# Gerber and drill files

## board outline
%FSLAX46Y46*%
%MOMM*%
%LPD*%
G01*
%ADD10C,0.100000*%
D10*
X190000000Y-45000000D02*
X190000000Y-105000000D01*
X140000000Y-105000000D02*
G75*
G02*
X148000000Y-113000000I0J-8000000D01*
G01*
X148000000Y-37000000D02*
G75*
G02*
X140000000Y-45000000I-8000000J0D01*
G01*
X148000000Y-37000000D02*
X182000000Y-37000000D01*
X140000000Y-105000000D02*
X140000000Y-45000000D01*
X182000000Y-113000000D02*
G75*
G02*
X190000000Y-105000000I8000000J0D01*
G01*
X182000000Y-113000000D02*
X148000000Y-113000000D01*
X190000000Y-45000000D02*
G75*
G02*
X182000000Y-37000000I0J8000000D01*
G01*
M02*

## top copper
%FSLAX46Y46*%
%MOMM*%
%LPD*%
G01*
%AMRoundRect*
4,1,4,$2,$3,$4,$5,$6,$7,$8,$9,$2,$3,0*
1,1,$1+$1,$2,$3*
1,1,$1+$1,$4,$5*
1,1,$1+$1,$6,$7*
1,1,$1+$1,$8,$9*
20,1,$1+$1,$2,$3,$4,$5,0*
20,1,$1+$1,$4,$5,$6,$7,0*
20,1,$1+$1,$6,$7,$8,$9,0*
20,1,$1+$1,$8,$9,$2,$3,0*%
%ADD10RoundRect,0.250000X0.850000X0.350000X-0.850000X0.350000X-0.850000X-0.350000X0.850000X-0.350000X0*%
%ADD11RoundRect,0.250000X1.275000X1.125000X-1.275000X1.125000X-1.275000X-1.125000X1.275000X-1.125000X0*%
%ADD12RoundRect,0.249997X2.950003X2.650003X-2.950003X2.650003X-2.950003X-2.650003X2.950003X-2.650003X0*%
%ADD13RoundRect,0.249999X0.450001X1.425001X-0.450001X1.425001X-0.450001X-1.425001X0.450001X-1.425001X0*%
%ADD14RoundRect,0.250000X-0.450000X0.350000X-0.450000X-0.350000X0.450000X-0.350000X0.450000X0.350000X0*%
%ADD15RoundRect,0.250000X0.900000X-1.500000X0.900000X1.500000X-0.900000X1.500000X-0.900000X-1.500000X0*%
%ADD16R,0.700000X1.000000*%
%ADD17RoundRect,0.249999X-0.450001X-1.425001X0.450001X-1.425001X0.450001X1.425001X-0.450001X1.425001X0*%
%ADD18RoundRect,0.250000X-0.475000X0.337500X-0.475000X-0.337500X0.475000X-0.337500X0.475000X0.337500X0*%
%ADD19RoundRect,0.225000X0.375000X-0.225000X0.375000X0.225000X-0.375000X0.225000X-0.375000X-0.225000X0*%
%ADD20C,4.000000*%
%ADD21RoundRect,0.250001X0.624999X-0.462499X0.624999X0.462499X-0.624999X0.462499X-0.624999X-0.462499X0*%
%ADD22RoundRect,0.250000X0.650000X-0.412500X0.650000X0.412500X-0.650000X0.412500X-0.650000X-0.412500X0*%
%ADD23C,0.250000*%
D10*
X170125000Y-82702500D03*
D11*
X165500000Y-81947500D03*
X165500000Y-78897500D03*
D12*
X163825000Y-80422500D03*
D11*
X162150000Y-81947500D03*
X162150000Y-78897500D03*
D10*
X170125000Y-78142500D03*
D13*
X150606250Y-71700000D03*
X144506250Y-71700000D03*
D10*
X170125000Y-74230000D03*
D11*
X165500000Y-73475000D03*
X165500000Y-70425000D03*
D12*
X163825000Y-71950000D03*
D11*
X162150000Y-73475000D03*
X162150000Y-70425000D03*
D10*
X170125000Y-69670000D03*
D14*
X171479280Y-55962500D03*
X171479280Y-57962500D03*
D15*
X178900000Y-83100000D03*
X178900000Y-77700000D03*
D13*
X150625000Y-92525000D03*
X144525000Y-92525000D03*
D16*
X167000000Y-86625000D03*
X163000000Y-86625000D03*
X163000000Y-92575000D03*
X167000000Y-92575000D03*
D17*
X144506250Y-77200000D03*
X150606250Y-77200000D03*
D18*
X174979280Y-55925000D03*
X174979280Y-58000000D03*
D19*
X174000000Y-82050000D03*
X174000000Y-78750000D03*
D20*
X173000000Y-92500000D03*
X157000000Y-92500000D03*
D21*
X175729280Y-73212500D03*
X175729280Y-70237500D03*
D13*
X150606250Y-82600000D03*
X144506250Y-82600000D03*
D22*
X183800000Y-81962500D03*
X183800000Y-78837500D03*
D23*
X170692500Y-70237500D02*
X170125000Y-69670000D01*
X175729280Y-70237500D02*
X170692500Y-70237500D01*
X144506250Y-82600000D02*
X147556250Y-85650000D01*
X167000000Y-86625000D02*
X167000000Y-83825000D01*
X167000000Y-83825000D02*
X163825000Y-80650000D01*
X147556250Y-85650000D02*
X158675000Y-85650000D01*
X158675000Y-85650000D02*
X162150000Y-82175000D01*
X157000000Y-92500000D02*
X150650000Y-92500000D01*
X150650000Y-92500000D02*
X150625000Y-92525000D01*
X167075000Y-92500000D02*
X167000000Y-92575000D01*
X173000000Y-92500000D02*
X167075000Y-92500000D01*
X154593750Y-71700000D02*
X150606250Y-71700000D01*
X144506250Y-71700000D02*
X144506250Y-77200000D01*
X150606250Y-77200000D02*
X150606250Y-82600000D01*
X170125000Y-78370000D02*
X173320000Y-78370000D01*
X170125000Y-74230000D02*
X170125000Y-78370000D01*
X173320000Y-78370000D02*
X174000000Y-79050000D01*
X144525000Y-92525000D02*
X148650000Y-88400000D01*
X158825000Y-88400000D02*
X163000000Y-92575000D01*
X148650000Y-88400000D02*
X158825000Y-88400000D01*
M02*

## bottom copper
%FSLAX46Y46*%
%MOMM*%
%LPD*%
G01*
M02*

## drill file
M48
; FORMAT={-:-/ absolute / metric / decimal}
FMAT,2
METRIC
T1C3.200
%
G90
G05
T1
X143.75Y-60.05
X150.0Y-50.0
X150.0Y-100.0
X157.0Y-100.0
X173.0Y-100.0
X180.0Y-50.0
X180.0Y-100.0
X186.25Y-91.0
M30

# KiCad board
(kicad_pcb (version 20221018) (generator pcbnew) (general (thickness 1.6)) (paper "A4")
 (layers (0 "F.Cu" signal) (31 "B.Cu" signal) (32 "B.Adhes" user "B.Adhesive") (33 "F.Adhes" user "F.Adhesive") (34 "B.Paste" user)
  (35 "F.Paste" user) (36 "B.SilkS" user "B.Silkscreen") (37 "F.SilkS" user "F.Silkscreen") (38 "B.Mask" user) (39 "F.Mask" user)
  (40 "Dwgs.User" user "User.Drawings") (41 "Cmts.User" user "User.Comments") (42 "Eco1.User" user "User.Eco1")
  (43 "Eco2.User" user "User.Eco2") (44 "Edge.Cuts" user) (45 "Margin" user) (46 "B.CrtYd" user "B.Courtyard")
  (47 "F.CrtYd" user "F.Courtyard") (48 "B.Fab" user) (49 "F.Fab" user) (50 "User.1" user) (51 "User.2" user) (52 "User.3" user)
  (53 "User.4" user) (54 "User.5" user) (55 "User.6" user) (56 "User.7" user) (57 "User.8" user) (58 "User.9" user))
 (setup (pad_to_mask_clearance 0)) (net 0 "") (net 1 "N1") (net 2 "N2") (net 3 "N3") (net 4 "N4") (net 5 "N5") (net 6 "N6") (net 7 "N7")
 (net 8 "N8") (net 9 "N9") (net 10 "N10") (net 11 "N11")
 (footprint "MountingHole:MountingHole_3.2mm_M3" (layer "F.Cu") (at 186.25 91)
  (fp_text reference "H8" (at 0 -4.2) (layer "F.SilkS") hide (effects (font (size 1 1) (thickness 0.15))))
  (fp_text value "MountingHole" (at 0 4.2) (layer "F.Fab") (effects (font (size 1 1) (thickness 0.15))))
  (pad "" np_thru_hole circle (at 0 0) (size 3.2 3.2) (drill 3.2) (layers "*.Cu" "*.Mask")))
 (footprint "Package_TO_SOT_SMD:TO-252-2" (layer "F.Cu") (at 165.085 80.4225 180)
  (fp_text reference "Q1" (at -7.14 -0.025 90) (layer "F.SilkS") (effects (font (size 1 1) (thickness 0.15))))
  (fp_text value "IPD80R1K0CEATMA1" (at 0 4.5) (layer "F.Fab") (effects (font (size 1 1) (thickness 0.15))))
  (pad "1" smd roundrect (at -5.04 -2.28 180) (size 2.2 1.2) (layers "F.Cu" "F.Paste" "F.Mask") (roundrect_rratio 0.2083333333) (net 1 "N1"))
  (pad "2" smd roundrect (at -0.415 -1.525 180) (size 3.05 2.75) (layers "F.Cu" "F.Paste") (roundrect_rratio 0.09090909091) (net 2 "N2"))
  (pad "2" smd roundrect (at -0.415 1.525 180) (size 3.05 2.75) (layers "F.Cu" "F.Paste") (roundrect_rratio 0.09090909091) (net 2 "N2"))
  (pad "2" smd roundrect (at 1.26 0 180) (size 6.4 5.8) (layers "F.Cu" "F.Mask") (roundrect_rratio 0.04310293103) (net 2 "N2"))
  (pad "2" smd roundrect (at 2.935 -1.525 180) (size 3.05 2.75) (layers "F.Cu" "F.Paste") (roundrect_rratio 0.09090909091) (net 2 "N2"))
  (pad "2" smd roundrect (at 2.935 1.525 180) (size 3.05 2.75) (layers "F.Cu" "F.Paste") (roundrect_rratio 0.09090909091) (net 2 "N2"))
  (pad "3" smd roundrect (at -5.04 2.28 180) (size 2.2 1.2) (layers "F.Cu" "F.Paste" "F.Mask") (roundrect_rratio 0.2083333333) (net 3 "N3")))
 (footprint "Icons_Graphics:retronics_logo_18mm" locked (layer "F.Cu") (at 165 105)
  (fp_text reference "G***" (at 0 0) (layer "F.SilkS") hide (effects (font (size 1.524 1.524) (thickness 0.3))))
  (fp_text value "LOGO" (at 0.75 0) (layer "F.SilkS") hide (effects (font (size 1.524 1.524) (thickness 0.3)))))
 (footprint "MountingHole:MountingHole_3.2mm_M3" (layer "F.Cu") (at 150 100)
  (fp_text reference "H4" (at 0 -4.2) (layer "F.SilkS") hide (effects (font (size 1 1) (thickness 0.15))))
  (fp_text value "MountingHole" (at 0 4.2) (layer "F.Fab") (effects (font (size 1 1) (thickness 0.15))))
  (pad "" np_thru_hole circle (at 0 0) (size 3.2 3.2) (drill 3.2) (layers "*.Cu" "*.Mask")))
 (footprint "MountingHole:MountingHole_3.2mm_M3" (layer "F.Cu") (at 180 50)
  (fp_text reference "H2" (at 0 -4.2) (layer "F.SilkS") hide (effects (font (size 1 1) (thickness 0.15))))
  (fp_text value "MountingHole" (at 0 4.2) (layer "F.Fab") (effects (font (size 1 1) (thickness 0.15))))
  (pad "" np_thru_hole circle (at 0 0) (size 3.2 3.2) (drill 3.2) (layers "*.Cu" "*.Mask")))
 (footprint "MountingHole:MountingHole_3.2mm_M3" (layer "F.Cu") (at 157 100)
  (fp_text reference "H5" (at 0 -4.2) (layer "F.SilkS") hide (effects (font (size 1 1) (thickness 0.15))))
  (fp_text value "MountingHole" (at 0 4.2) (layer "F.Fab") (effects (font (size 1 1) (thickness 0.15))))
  (pad "" np_thru_hole circle (at 0 0) (size 3.2 3.2) (drill 3.2) (layers "*.Cu" "*.Mask")))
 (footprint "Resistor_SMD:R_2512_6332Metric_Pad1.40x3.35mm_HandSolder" (layer "F.Cu") (at 147.55625 71.7 180)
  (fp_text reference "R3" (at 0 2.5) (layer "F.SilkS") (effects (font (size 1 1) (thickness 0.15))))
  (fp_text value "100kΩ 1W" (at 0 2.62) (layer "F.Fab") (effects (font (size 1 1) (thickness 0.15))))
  (pad "1" smd roundrect (at -3.05 0 180) (size 1.4 3.35) (layers "F.Cu" "F.Paste" "F.Mask") (roundrect_rratio 0.1785707143) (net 1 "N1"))
  (pad "2" smd roundrect (at 3.05 0 180) (size 1.4 3.35) (layers "F.Cu" "F.Paste" "F.Mask") (roundrect_rratio 0.1785707143) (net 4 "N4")))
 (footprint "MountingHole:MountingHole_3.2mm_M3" (layer "F.Cu") (at 180 100)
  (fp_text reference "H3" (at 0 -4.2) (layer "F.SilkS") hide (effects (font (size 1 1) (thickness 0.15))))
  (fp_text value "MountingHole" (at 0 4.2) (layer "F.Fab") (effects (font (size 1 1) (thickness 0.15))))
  (pad "" np_thru_hole circle (at 0 0) (size 3.2 3.2) (drill 3.2) (layers "*.Cu" "*.Mask")))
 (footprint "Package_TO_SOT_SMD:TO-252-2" (layer "F.Cu") (at 165.085 71.95 180)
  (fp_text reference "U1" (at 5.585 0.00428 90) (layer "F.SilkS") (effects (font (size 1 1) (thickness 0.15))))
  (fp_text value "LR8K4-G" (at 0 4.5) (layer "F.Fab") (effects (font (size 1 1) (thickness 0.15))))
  (pad "1" smd roundrect (at -5.04 -2.28 180) (size 2.2 1.2) (layers "F.Cu" "F.Paste" "F.Mask") (roundrect_rratio 0.2083333333) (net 3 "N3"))
  (pad "2" smd roundrect (at -0.415 -1.525 180) (size 3.05 2.75) (layers "F.Cu" "F.Paste") (roundrect_rratio 0.09090909091) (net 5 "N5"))
  (pad "2" smd roundrect (at -0.415 1.525 180) (size 3.05 2.75) (layers "F.Cu" "F.Paste") (roundrect_rratio 0.09090909091) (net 5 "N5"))
  (pad "2" smd roundrect (at 1.26 0 180) (size 6.4 5.8) (layers "F.Cu" "F.Mask") (roundrect_rratio 0.04310293103) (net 5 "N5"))
  (pad "2" smd roundrect (at 2.935 -1.525 180) (size 3.05 2.75) (layers "F.Cu" "F.Paste") (roundrect_rratio 0.09090909091) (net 5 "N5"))
  (pad "2" smd roundrect (at 2.935 1.525 180) (size 3.05 2.75) (layers "F.Cu" "F.Paste") (roundrect_rratio 0.09090909091) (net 5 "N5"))
  (pad "3" smd roundrect (at -5.04 2.28 180) (size 2.2 1.2) (layers "F.Cu" "F.Paste" "F.Mask") (roundrect_rratio 0.2083333333) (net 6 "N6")))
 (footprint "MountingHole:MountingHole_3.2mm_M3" (layer "F.Cu") (at 143.75 60.05)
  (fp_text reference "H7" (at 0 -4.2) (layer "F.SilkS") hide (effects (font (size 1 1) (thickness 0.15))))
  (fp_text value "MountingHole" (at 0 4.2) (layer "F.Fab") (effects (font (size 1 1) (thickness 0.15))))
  (pad "" np_thru_hole circle (at 0 0) (size 3.2 3.2) (drill 3.2) (layers "*.Cu" "*.Mask")))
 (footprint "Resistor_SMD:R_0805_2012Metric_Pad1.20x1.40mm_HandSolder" (layer "F.Cu") (at 171.47928 56.9625 -90)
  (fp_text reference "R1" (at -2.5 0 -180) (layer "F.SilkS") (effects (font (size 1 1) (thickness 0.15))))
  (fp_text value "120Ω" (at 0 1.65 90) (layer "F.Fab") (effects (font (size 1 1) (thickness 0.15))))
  (pad "1" smd roundrect (at -1 0 270) (size 1.2 1.4) (layers "F.Cu" "F.Paste" "F.Mask") (roundrect_rratio 0.2083333333) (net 5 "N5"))
  (pad "2" smd roundrect (at 1 0 270) (size 1.2 1.4) (layers "F.Cu" "F.Paste" "F.Mask") (roundrect_rratio 0.2083333333) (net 6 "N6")))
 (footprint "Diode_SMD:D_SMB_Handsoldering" (layer "F.Cu") (at 178.9 80.4 90)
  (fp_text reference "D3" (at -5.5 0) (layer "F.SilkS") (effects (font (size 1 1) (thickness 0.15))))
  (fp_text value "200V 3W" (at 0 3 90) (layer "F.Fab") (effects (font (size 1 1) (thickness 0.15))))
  (pad "1" smd roundrect (at -2.7 0 90) (size 3.5 2.3) (layers "F.Cu" "F.Paste" "F.Mask") (roundrect_rratio 0.1086956522) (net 1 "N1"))
  (pad "2" smd roundrect (at 2.7 0 90) (size 3.5 2.3) (layers "F.Cu" "F.Paste" "F.Mask") (roundrect_rratio 0.1086956522) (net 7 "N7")))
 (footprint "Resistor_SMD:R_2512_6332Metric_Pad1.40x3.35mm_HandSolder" (layer "F.Cu") (at 147.575 92.525 180)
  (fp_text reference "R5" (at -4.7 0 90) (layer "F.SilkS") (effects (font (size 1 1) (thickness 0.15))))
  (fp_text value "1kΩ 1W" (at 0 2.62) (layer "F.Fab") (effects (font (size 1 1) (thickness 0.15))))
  (pad "1" smd roundrect (at -3.05 0 180) (size 1.4 3.35) (layers "F.Cu" "F.Paste" "F.Mask") (roundrect_rratio 0.178571) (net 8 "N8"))
  (pad "2" smd roundrect (at 3.05 0 180) (size 1.4 3.35) (layers "F.Cu" "F.Paste" "F.Mask") (roundrect_rratio 0.178571) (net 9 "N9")))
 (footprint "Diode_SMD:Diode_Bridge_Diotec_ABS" (layer "F.Cu") (at 165 89.6 -90)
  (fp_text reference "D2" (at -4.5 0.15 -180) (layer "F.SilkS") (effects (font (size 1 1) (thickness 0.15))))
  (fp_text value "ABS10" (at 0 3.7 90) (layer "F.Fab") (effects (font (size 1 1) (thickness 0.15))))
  (pad "1" smd rect (at -2.975 -2 270) (size 1 0.7) (layers "F.Cu" "F.Paste" "F.Mask") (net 2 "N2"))
  (pad "2" smd rect (at -2.975 2 270) (size 1 0.7) (layers "F.Cu" "F.Paste" "F.Mask") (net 7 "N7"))
  (pad "3" smd rect (at 2.975 2 270) (size 1 0.7) (layers "F.Cu" "F.Paste" "F.Mask") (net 9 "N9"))
  (pad "4" smd rect (at 2.975 -2 270) (size 1 0.7) (layers "F.Cu" "F.Paste" "F.Mask") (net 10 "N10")))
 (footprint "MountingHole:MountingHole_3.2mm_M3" (layer "F.Cu") (at 173 100)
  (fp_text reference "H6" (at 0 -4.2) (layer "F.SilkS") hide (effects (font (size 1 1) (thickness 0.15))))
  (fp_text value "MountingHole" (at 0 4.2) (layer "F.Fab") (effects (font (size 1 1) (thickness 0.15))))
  (pad "" np_thru_hole circle (at 0 0) (size 3.2 3.2) (drill 3.2) (layers "*.Cu" "*.Mask")))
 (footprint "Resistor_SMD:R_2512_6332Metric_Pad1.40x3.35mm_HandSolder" (layer "F.Cu") (at 147.55625 77.2)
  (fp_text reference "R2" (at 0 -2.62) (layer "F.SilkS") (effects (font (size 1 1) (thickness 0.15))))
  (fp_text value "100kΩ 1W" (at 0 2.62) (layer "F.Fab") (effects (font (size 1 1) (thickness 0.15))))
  (pad "1" smd roundrect (at -3.05 0) (size 1.4 3.35) (layers "F.Cu" "F.Paste" "F.Mask") (roundrect_rratio 0.1785707143) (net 4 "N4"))
  (pad "2" smd roundrect (at 3.05 0) (size 1.4 3.35) (layers "F.Cu" "F.Paste" "F.Mask") (roundrect_rratio 0.1785707143) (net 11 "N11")))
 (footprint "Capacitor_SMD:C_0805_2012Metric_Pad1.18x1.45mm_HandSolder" (layer "F.Cu") (at 174.97928 56.9625 -90)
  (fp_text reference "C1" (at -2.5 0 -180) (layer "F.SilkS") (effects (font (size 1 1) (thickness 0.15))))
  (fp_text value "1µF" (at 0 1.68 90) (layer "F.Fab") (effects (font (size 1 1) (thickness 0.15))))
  (pad "1" smd roundrect (at -1.0375 0 270) (size 1.175 1.45) (layers "F.Cu" "F.Paste" "F.Mask") (roundrect_rratio 0.2127659574)
   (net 5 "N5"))
  (pad "2" smd roundrect (at 1.0375 0 270) (size 1.175 1.45) (layers "F.Cu" "F.Paste" "F.Mask") (roundrect_rratio 0.2127659574) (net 7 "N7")))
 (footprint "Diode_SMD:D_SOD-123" (layer "F.Cu") (at 174 80.4 90)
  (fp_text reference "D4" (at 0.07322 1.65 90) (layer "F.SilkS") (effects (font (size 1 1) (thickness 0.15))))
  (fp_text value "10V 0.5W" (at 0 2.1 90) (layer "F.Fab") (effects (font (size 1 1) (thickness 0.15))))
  (pad "1" smd roundrect (at -1.65 0 90) (size 0.9 1.2) (layers "F.Cu" "F.Paste" "F.Mask") (roundrect_rratio 0.25) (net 1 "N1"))
  (pad "2" smd roundrect (at 1.65 0 90) (size 0.9 1.2) (layers "F.Cu" "F.Paste" "F.Mask") (roundrect_rratio 0.25) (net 3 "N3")))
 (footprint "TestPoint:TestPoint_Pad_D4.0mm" (layer "F.Cu") (at 173 92.5)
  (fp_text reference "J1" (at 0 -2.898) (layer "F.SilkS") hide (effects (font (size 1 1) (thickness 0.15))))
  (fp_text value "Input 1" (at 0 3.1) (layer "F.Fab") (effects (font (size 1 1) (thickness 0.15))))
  (pad "1" smd circle (at 0 0) (size 4 4) (layers "F.Cu" "F.Mask") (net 10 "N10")))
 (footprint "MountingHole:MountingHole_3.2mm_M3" (layer "F.Cu") (at 150 50)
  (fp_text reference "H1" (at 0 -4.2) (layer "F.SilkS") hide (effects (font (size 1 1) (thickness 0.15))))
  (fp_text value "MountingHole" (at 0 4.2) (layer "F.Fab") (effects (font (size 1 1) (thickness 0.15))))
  (pad "" np_thru_hole circle (at 0 0) (size 3.2 3.2) (drill 3.2) (layers "*.Cu" "*.Mask")))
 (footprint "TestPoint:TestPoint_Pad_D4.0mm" (layer "F.Cu") (at 157 92.5)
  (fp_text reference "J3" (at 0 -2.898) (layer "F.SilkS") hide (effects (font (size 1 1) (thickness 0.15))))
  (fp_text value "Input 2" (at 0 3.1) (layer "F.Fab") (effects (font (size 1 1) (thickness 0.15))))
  (pad "1" smd circle (at 0 0) (size 4 4) (layers "F.Cu" "F.Mask") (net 8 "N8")))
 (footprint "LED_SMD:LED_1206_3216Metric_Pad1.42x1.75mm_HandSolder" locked (layer "F.Cu") (at 175.72928 71.725 90)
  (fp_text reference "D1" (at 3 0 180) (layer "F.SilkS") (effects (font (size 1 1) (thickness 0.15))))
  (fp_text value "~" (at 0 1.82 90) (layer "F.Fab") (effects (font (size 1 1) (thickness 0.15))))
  (pad "1" smd roundrect locked (at -1.4875 0 90) (size 1.425 1.75) (layers "F.Cu" "F.Paste" "F.Mask") (roundrect_rratio 0.1754392982)
   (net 7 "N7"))
  (pad "2" smd roundrect locked (at 1.4875 0 90) (size 1.425 1.75) (layers "F.Cu" "F.Paste" "F.Mask") (roundrect_rratio 0.1754392982)
   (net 6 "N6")))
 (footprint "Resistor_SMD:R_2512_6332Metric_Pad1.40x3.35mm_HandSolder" (layer "F.Cu") (at 147.55625 82.6 180)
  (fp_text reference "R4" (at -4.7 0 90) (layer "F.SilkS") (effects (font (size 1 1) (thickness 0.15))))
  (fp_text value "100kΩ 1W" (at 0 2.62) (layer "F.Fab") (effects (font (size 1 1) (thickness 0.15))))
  (pad "1" smd roundrect (at -3.05 0 180) (size 1.4 3.35) (layers "F.Cu" "F.Paste" "F.Mask") (roundrect_rratio 0.1785707143) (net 11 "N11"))
  (pad "2" smd roundrect (at 3.05 0 180) (size 1.4 3.35) (layers "F.Cu" "F.Paste" "F.Mask") (roundrect_rratio 0.1785707143) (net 2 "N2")))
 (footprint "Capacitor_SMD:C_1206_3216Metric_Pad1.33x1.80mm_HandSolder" (layer "F.Cu") (at 183.8 80.4 90)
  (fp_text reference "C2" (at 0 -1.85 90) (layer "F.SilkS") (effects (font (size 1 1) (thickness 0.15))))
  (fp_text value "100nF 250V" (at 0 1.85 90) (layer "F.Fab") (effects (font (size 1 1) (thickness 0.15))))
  (pad "1" smd roundrect (at -1.5625 0 90) (size 1.325 1.8) (layers "F.Cu" "F.Paste" "F.Mask") (roundrect_rratio 0.188679) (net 1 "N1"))
  (pad "2" smd roundrect (at 1.5625 0 90) (size 1.325 1.8) (layers "F.Cu" "F.Paste" "F.Mask") (roundrect_rratio 0.188679) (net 7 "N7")))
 (gr_line (start 190 45) (end 190 105) (stroke (width 0.1) (type default)) (layer "Edge.Cuts"))
 (gr_arc (start 140 105) (mid 145.656854 107.343146) (end 148 113) (stroke (width 0.1) (type default)) (layer "Edge.Cuts"))
 (gr_arc (start 148 37) (mid 145.656854 42.656854) (end 140 45) (stroke (width 0.1) (type default)) (layer "Edge.Cuts"))
 (gr_line (start 148 37) (end 182 37) (stroke (width 0.1) (type default)) (layer "Edge.Cuts"))
 (gr_line (start 140 105) (end 140 45) (stroke (width 0.1) (type default)) (layer "Edge.Cuts"))
 (gr_arc (start 182 113) (mid 184.343146 107.343146) (end 190 105) (stroke (width 0.1) (type default)) (layer "Edge.Cuts"))
 (gr_line (start 182 113) (end 148 113) (stroke (width 0.1) (type default)) (layer "Edge.Cuts"))
 (gr_arc (start 190 45) (mid 184.343146 42.656854) (end 182 37) (stroke (width 0.1) (type default)) (layer "Edge.Cuts"))
 (segment (start 170.6925 70.2375) (end 170.125 69.67) (width 0.25) (layer "F.Cu") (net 6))
 (segment (start 175.72928 70.2375) (end 170.6925 70.2375) (width 0.25) (layer "F.Cu") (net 6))
 (segment (start 144.50625 82.6) (end 147.55625 85.65) (width 0.25) (layer "F.Cu") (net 2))
 (segment (start 167 86.625) (end 167 83.825) (width 0.25) (layer "F.Cu") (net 2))
 (segment (start 167 83.825) (end 163.825 80.65) (width 0.25) (layer "F.Cu") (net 2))
 (segment (start 147.55625 85.65) (end 158.675 85.65) (width 0.25) (layer "F.Cu") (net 2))
 (segment (start 158.675 85.65) (end 162.15 82.175) (width 0.25) (layer "F.Cu") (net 2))
 (segment (start 157 92.5) (end 150.65 92.5) (width 0.25) (layer "F.Cu") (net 8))
 (segment (start 150.65 92.5) (end 150.625 92.525) (width 0.25) (layer "F.Cu") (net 8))
 (segment (start 167.075 92.5) (end 167 92.575) (width 0.25) (layer "F.Cu") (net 10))
 (segment (start 173 92.5) (end 167.075 92.5) (width 0.25) (layer "F.Cu") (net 10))
 (segment (start 154.59375 71.7) (end 150.60625 71.7) (width 0.25) (layer "F.Cu") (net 1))
 (segment (start 144.50625 71.7) (end 144.50625 77.2) (width 0.25) (layer "F.Cu") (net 4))
 (segment (start 150.60625 77.2) (end 150.60625 82.6) (width 0.25) (layer "F.Cu") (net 11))
 (segment (start 170.125 78.37) (end 173.32 78.37) (width 0.25) (layer "F.Cu") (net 3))
 (segment (start 170.125 74.23) (end 170.125 78.37) (width 0.25) (layer "F.Cu") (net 3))
 (segment (start 173.32 78.37) (end 174 79.05) (width 0.25) (layer "F.Cu") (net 3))
 (segment (start 144.525 92.525) (end 148.65 88.4) (width 0.25) (layer "F.Cu") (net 9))
 (segment (start 158.825 88.4) (end 163 92.575) (width 0.25) (layer "F.Cu") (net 9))
 (segment (start 148.65 88.4) (end 158.825 88.4) (width 0.25) (layer "F.Cu") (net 9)))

